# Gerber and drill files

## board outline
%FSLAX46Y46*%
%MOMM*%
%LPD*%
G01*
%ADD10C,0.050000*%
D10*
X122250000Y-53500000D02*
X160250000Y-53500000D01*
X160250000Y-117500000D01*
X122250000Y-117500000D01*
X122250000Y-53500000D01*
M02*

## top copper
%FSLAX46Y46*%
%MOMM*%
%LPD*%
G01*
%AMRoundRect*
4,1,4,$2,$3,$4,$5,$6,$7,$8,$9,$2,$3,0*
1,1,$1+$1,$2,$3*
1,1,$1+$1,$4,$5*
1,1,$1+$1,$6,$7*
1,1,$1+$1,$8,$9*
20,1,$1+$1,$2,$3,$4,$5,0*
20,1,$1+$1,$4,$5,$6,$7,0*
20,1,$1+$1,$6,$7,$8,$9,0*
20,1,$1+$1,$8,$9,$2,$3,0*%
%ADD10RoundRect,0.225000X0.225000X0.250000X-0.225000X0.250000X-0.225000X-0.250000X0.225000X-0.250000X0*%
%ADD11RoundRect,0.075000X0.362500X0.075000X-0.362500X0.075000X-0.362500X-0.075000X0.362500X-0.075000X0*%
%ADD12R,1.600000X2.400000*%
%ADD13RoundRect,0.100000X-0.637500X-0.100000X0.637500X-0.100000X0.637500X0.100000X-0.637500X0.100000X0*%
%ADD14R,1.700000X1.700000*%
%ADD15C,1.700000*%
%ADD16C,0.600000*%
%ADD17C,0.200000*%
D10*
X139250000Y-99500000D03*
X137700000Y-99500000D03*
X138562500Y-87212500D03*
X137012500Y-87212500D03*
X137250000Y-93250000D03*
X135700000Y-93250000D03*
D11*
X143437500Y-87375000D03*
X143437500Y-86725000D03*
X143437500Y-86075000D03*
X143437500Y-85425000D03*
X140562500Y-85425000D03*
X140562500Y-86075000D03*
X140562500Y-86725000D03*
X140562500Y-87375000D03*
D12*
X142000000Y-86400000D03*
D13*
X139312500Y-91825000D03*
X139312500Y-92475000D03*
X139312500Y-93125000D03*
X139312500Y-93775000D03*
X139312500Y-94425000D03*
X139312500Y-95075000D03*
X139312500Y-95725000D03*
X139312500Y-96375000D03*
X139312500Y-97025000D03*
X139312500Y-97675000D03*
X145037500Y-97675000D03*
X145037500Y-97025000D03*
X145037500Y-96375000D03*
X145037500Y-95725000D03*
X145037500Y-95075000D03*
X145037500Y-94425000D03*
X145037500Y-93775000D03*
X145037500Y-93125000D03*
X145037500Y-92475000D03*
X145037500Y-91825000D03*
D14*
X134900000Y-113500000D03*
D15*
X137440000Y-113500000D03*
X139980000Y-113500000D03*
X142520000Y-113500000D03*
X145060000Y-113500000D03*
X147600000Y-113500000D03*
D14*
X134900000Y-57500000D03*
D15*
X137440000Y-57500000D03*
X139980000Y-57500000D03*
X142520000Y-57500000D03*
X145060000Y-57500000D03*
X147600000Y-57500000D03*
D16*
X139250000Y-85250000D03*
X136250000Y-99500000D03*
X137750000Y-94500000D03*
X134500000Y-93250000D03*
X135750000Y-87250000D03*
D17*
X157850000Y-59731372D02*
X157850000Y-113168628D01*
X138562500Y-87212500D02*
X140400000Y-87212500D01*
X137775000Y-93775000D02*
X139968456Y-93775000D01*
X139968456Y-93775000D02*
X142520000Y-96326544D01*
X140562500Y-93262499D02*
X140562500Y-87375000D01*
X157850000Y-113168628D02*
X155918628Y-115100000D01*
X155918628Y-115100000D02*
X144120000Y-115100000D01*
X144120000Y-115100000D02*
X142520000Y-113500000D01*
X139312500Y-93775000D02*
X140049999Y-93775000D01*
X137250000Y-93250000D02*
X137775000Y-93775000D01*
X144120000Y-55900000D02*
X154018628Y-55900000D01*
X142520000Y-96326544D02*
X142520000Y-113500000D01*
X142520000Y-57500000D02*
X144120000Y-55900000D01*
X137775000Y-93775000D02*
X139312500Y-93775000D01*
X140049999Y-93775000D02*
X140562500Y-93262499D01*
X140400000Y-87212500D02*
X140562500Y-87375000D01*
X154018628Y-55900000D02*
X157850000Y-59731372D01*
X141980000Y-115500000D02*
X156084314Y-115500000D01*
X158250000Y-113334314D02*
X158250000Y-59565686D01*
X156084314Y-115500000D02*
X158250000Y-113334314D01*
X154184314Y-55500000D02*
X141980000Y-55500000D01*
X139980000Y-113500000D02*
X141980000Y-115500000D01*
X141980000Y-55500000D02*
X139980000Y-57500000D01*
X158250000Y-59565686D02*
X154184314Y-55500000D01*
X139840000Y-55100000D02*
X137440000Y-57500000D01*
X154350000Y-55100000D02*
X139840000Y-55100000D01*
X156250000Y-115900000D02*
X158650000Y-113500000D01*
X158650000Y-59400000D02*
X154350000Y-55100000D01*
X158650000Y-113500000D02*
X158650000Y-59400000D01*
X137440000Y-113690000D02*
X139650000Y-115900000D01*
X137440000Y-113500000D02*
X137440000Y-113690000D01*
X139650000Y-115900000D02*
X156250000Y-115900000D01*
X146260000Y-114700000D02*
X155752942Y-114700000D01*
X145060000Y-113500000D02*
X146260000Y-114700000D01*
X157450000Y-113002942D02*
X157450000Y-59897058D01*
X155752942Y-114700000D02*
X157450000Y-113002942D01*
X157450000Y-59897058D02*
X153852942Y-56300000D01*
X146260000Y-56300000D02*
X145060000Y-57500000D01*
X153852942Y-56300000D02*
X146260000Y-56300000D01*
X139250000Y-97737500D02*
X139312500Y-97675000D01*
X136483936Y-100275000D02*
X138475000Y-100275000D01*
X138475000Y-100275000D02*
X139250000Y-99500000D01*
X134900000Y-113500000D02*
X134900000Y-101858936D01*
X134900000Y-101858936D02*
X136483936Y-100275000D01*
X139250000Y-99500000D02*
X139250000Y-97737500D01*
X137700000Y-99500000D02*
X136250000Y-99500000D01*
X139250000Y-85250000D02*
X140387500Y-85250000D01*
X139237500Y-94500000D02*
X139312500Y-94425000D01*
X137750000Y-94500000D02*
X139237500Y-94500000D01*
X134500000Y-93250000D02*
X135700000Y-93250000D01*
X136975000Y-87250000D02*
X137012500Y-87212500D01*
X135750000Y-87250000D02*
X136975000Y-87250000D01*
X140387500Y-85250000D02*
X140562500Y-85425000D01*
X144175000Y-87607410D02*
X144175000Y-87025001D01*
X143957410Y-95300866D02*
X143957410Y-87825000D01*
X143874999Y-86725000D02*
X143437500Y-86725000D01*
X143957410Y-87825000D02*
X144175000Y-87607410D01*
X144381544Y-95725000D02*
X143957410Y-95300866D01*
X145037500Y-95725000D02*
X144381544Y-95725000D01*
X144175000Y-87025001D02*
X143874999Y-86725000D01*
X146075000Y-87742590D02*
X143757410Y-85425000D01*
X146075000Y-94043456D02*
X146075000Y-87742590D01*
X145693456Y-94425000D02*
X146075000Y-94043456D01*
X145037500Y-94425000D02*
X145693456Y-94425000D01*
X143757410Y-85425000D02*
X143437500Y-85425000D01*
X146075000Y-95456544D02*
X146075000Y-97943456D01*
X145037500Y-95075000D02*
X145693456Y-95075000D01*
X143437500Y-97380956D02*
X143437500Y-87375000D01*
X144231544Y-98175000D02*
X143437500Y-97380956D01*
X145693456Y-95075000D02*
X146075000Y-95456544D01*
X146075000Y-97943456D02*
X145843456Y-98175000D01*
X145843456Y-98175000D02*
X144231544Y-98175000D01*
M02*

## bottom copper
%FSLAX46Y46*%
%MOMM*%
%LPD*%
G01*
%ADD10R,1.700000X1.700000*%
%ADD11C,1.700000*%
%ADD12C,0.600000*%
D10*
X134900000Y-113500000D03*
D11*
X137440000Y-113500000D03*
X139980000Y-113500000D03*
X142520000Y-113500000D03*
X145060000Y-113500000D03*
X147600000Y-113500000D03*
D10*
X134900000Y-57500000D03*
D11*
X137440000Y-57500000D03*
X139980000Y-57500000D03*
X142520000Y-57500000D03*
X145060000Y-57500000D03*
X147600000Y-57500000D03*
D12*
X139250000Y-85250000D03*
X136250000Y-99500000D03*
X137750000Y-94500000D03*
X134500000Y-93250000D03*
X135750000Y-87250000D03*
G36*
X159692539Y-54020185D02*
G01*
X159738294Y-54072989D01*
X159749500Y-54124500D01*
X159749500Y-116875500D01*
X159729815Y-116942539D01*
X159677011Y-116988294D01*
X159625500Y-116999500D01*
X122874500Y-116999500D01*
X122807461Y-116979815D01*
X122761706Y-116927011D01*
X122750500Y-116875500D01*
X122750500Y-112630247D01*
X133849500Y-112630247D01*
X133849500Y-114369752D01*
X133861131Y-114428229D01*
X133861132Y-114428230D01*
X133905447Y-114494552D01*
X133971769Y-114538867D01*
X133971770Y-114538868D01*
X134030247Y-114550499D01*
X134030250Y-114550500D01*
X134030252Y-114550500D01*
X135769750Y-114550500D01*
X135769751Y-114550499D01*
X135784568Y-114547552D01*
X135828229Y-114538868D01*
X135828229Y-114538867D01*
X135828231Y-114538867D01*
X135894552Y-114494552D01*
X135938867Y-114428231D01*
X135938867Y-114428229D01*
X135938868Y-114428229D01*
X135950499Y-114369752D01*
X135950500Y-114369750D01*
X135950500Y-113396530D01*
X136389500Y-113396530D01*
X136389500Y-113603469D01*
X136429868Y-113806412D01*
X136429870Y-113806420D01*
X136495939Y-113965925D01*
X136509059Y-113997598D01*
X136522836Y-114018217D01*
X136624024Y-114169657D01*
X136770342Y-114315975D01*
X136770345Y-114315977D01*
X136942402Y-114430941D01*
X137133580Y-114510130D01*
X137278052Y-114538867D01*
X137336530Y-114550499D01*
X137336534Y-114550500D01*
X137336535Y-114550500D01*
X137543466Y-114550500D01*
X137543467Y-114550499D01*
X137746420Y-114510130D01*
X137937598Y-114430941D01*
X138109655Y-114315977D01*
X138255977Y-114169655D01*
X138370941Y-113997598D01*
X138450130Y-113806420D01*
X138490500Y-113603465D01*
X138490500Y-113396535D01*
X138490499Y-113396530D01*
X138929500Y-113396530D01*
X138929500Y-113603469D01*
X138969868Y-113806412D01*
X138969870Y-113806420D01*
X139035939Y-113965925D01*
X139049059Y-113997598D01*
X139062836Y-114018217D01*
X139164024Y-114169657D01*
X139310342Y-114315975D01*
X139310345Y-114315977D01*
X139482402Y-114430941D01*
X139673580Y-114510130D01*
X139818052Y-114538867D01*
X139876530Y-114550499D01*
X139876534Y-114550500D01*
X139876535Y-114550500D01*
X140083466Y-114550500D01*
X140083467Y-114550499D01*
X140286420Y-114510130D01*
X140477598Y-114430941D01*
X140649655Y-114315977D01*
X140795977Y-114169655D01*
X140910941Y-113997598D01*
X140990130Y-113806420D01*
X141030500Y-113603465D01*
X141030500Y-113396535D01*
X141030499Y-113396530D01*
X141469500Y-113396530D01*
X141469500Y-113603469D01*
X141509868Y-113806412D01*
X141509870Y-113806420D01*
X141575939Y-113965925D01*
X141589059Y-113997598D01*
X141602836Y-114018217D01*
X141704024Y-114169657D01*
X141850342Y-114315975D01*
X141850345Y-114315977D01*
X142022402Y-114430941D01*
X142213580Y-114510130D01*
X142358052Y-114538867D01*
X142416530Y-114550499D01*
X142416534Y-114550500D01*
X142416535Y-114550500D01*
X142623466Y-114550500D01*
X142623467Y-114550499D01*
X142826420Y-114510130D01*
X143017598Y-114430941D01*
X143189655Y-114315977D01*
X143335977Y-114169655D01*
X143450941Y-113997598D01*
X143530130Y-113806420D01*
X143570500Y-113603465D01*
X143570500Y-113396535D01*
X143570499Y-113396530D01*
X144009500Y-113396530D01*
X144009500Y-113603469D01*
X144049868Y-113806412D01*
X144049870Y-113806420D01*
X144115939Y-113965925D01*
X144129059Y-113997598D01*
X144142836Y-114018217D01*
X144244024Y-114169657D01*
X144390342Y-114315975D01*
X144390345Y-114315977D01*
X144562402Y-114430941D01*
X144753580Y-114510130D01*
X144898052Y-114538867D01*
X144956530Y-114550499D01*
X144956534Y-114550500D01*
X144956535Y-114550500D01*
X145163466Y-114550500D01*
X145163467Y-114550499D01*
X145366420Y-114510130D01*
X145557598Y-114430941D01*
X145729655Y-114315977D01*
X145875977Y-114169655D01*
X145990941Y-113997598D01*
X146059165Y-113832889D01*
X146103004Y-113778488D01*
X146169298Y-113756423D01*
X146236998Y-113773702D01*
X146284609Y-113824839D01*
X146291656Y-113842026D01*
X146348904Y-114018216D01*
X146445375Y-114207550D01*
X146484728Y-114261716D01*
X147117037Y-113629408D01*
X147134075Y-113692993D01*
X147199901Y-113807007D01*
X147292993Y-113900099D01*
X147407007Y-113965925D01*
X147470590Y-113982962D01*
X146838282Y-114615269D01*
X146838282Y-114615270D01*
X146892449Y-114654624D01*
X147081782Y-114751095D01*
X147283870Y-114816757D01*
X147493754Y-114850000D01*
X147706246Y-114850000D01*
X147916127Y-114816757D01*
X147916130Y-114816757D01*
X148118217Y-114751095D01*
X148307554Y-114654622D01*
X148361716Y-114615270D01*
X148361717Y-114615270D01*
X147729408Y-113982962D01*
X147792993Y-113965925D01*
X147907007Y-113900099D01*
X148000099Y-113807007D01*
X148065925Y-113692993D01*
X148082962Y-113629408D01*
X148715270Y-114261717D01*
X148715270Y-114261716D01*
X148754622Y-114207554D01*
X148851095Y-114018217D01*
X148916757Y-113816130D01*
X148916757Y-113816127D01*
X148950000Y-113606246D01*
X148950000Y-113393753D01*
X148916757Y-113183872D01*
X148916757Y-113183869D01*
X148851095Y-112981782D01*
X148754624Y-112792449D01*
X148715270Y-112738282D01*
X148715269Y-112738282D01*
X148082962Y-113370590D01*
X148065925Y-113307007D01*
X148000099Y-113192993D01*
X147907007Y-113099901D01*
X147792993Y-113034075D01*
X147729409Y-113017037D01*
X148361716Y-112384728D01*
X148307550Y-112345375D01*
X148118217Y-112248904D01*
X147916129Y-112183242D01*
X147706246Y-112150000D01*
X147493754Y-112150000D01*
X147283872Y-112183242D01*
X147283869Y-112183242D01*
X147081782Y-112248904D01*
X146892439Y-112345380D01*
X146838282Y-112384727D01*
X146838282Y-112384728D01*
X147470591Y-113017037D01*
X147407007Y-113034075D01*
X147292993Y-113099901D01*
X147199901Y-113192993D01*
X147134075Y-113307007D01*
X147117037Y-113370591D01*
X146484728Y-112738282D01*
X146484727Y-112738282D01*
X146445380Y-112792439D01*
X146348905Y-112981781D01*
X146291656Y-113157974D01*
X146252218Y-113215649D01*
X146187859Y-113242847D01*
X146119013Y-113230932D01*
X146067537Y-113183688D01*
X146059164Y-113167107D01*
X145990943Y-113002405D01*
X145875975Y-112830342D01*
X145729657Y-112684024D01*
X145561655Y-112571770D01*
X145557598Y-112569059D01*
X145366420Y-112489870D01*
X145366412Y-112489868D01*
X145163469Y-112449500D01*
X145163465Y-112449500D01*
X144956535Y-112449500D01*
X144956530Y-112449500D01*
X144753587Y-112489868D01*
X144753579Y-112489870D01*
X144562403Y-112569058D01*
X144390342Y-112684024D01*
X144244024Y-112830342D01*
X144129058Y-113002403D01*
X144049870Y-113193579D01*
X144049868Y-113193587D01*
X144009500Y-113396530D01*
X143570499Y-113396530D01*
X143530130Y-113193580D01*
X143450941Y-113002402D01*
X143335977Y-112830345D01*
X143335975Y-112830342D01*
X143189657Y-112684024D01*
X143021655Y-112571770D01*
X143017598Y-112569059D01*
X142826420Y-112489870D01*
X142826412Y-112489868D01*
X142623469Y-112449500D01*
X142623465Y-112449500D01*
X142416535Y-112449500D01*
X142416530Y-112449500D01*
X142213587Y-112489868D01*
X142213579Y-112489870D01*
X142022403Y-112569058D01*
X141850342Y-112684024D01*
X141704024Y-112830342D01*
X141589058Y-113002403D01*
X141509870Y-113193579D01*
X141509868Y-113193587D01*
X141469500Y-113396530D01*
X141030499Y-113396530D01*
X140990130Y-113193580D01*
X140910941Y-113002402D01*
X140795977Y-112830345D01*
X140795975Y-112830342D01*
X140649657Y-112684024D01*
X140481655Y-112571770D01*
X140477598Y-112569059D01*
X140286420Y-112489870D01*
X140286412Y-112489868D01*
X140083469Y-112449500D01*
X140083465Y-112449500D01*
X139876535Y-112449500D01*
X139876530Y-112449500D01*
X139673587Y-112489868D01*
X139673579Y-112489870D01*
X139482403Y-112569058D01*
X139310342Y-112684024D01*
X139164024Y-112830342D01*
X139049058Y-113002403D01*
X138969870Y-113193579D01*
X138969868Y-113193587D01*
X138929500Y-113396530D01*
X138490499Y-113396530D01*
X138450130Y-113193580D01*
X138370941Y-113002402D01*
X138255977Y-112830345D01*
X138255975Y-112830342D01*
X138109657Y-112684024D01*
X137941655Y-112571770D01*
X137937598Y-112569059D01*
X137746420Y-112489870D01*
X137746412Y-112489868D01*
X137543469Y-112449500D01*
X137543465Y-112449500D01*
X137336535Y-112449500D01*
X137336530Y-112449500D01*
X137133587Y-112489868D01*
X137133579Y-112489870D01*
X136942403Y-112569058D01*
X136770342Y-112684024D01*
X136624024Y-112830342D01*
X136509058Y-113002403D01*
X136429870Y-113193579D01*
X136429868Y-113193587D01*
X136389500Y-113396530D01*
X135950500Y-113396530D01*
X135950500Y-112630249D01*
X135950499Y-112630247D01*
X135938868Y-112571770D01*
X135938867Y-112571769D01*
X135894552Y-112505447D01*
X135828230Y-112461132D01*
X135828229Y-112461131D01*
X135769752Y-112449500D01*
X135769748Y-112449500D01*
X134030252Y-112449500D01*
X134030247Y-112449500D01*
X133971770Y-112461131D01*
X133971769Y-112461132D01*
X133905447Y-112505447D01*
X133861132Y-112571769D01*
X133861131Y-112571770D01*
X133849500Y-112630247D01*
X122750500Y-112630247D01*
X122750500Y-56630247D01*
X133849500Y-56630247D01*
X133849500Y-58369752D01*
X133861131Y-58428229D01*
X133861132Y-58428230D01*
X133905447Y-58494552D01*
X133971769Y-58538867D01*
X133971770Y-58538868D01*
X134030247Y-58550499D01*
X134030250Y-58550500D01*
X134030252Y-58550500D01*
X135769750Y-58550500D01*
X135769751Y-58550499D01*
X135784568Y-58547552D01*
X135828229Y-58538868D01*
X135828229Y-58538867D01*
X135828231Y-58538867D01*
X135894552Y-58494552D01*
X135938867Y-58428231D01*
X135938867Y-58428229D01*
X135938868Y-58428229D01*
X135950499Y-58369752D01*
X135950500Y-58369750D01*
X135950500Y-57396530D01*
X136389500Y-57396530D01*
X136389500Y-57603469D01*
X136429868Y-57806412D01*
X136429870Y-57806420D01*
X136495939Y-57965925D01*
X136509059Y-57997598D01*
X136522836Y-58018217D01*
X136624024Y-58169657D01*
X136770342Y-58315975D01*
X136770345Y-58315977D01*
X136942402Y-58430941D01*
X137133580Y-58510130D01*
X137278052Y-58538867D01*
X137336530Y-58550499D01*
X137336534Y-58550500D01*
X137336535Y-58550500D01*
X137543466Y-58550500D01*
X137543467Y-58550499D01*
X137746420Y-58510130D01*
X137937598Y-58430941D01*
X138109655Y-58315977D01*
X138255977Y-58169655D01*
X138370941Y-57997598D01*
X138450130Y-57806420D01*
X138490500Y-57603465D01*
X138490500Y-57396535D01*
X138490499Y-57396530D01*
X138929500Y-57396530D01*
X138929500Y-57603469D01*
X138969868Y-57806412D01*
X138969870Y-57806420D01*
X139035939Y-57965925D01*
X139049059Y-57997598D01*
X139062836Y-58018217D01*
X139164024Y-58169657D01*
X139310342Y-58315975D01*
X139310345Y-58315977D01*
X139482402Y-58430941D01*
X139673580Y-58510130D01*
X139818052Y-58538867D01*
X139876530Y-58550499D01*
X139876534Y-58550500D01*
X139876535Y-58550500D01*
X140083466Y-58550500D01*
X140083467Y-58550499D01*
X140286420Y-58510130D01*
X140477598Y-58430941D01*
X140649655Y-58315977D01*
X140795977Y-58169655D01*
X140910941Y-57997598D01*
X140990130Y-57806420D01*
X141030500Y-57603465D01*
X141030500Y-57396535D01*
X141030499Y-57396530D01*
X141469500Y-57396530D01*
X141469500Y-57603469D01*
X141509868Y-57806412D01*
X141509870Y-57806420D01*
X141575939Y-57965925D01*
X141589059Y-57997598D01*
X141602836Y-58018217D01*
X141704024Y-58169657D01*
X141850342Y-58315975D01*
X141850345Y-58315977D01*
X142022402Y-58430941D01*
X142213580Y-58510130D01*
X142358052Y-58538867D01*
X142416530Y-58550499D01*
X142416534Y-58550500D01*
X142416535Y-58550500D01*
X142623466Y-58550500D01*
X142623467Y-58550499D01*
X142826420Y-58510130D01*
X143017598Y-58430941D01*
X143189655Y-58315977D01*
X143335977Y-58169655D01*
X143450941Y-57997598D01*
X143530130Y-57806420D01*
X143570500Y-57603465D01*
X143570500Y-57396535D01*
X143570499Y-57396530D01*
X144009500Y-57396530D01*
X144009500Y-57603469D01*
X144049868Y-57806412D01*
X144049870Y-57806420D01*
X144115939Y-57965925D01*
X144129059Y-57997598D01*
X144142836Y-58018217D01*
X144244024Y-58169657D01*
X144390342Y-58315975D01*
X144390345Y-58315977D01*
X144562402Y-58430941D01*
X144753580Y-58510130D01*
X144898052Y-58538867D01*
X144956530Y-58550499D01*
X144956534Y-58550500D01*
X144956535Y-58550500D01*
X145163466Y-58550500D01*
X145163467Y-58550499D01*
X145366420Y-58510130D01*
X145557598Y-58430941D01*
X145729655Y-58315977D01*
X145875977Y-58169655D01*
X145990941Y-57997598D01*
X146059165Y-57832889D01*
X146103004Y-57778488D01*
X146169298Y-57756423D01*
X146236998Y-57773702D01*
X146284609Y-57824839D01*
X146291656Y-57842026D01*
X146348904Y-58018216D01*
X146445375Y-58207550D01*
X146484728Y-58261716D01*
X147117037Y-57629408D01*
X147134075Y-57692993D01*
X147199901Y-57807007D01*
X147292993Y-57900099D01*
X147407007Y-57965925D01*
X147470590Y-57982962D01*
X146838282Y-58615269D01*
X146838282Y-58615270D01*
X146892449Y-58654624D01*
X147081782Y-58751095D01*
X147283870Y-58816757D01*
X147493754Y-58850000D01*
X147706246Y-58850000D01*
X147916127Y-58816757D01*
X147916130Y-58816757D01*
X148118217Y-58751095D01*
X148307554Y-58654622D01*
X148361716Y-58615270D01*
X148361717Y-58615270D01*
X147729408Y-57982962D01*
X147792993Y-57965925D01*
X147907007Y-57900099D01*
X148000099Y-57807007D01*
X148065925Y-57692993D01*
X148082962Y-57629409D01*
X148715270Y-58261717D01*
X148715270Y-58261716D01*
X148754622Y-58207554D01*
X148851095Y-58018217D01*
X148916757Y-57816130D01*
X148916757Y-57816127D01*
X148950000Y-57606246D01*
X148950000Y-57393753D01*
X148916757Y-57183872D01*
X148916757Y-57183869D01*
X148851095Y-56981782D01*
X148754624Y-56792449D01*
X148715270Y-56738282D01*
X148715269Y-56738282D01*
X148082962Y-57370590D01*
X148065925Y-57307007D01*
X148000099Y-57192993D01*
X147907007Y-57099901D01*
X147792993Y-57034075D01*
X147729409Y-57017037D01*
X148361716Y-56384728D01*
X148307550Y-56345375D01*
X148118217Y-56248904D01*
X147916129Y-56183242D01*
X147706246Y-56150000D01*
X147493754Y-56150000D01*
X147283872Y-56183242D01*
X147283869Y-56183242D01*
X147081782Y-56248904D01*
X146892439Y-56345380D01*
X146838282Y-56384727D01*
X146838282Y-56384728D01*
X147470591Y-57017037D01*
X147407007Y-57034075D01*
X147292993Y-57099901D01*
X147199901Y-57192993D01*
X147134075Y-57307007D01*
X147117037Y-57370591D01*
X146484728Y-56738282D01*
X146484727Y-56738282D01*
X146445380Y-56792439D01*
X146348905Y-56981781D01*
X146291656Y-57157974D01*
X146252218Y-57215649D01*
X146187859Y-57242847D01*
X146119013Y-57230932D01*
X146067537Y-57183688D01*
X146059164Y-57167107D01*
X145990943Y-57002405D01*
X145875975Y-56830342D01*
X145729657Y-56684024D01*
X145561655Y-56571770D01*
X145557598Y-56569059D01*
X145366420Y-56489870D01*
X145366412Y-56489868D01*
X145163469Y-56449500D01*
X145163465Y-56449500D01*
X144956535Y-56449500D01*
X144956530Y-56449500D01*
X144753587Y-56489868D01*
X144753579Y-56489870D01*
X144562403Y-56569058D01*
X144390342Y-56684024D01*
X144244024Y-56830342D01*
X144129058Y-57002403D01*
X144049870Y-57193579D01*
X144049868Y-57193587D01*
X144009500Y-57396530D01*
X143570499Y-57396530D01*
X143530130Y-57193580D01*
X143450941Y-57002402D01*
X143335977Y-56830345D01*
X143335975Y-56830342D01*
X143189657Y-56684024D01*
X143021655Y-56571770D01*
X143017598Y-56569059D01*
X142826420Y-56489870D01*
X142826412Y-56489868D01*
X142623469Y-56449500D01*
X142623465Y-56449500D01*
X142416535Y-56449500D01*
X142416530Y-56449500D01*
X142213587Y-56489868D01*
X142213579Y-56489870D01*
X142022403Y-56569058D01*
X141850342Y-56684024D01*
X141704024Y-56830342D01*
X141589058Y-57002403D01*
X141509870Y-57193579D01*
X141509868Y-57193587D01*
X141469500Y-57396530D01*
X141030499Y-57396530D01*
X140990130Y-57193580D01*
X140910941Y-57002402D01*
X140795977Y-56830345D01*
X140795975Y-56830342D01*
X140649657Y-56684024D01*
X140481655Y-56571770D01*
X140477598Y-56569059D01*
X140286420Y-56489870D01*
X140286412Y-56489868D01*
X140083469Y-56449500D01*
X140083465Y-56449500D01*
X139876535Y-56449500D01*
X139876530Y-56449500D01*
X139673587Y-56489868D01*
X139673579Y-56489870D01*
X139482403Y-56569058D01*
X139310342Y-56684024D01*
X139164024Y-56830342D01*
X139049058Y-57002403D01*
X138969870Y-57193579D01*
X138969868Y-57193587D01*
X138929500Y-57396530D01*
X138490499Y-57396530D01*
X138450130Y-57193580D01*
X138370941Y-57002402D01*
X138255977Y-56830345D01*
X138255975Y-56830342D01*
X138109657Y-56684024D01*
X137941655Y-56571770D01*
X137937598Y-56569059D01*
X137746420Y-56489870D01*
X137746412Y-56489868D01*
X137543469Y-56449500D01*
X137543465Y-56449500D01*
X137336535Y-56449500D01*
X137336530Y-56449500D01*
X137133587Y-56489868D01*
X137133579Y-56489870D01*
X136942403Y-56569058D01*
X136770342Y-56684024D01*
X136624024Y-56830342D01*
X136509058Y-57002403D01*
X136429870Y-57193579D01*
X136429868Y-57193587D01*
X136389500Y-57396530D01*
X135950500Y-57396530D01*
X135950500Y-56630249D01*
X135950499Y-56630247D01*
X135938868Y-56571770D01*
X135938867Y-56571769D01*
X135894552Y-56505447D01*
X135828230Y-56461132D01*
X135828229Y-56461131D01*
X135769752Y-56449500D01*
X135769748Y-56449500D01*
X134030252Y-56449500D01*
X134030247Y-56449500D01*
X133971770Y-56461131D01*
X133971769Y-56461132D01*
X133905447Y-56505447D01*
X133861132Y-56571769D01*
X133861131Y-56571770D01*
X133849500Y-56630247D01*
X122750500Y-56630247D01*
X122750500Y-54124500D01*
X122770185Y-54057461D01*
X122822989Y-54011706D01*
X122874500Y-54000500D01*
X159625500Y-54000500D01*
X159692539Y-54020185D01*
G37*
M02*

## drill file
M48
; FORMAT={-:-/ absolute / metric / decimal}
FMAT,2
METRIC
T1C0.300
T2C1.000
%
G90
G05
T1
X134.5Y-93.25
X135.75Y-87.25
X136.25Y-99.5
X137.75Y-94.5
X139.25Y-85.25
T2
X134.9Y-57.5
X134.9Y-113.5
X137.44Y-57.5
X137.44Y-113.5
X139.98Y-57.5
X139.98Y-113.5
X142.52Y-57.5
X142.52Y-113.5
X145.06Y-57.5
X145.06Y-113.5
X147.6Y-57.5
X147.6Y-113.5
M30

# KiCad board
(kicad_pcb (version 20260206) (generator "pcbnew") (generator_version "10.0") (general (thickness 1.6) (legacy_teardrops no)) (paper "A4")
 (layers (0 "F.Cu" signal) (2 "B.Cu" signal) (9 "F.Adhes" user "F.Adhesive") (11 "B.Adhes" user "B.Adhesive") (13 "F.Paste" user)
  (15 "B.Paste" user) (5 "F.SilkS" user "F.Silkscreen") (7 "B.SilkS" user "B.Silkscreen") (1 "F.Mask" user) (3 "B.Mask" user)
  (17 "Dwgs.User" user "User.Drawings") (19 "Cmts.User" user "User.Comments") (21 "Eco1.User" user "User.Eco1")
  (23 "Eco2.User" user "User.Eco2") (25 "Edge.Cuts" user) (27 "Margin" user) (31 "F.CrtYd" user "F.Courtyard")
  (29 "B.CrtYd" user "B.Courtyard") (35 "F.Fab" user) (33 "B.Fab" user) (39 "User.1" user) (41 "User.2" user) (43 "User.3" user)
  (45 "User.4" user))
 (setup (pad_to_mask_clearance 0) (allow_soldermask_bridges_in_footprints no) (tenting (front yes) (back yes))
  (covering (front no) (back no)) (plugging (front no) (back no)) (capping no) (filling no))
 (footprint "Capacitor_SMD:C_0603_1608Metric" (layer "F.Cu") (at 138.475 99.5 180)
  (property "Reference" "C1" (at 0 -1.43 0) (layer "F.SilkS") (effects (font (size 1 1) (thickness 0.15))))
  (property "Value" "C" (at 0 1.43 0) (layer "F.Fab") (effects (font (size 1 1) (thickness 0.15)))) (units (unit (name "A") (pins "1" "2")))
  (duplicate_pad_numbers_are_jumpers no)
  (pad "1" smd roundrect (at -0.775 0 180) (size 0.9 0.95) (layers "F.Cu" "F.Mask" "F.Paste") (roundrect_rratio 0.25) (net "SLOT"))
  (pad "2" smd roundrect (at 0.775 0 180) (size 0.9 0.95) (layers "F.Cu" "F.Mask" "F.Paste") (roundrect_rratio 0.25) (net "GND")))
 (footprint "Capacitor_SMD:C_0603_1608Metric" (layer "F.Cu") (at 137.7875 87.2125 180)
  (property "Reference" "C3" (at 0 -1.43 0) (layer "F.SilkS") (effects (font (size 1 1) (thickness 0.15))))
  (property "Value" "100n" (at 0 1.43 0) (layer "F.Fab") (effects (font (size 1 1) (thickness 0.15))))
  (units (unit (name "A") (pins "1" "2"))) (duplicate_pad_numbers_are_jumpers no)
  (pad "1" smd roundrect (at -0.775 0 180) (size 0.9 0.95) (layers "F.Cu" "F.Mask" "F.Paste") (roundrect_rratio 0.25) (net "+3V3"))
  (pad "2" smd roundrect (at 0.775 0 180) (size 0.9 0.95) (layers "F.Cu" "F.Mask" "F.Paste") (roundrect_rratio 0.25) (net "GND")))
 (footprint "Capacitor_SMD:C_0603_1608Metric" (layer "F.Cu") (at 136.475 93.25 180)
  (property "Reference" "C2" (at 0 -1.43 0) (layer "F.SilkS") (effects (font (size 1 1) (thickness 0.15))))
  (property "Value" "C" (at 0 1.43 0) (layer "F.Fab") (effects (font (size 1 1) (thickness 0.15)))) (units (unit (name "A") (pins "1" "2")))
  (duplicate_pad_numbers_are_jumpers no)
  (pad "1" smd roundrect (at -0.775 0 180) (size 0.9 0.95) (layers "F.Cu" "F.Mask" "F.Paste") (roundrect_rratio 0.25) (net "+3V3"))
  (pad "2" smd roundrect (at 0.775 0 180) (size 0.9 0.95) (layers "F.Cu" "F.Mask" "F.Paste") (roundrect_rratio 0.25) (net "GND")))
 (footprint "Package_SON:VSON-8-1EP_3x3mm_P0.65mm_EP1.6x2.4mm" (layer "F.Cu") (at 142 86.4 180)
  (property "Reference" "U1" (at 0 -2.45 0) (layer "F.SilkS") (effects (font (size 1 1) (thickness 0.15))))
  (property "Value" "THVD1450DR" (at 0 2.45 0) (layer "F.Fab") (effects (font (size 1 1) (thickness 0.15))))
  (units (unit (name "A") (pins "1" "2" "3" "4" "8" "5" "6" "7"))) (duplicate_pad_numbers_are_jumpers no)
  (pad "" smd roundrect (at 0 -0.6 180) (size 1.29 0.97) (layers "F.Paste") (roundrect_rratio 0.25))
  (pad "" smd roundrect (at 0 0.6 180) (size 1.29 0.97) (layers "F.Paste") (roundrect_rratio 0.25))
  (pad "1" smd roundrect (at -1.4375 -0.975 180) (size 0.875 0.3) (layers "F.Cu" "F.Mask" "F.Paste") (roundrect_rratio 0.25) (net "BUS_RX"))
  (pad "2" smd roundrect (at -1.4375 -0.325 180) (size 0.875 0.3) (layers "F.Cu" "F.Mask" "F.Paste") (roundrect_rratio 0.25) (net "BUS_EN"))
  (pad "3" smd roundrect (at -1.4375 0.325 180) (size 0.875 0.3) (layers "F.Cu" "F.Mask" "F.Paste") (roundrect_rratio 0.25) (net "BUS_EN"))
  (pad "4" smd roundrect (at -1.4375 0.975 180) (size 0.875 0.3) (layers "F.Cu" "F.Mask" "F.Paste") (roundrect_rratio 0.25) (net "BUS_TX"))
  (pad "5" smd roundrect (at 1.4375 0.975 180) (size 0.875 0.3) (layers "F.Cu" "F.Mask" "F.Paste") (roundrect_rratio 0.25) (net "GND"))
  (pad "6" smd roundrect (at 1.4375 0.325 180) (size 0.875 0.3) (layers "F.Cu" "F.Mask" "F.Paste") (roundrect_rratio 0.25) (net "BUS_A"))
  (pad "7" smd roundrect (at 1.4375 -0.325 180) (size 0.875 0.3) (layers "F.Cu" "F.Mask" "F.Paste") (roundrect_rratio 0.25) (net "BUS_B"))
  (pad "8" smd roundrect (at 1.4375 -0.975 180) (size 0.875 0.3) (layers "F.Cu" "F.Mask" "F.Paste") (roundrect_rratio 0.25) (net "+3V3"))
  (pad "9" smd rect (at 0 0 180) (size 1.6 2.4) (layers "F.Cu" "F.Mask") (zone_connect 2)))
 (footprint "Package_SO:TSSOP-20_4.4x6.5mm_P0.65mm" (layer "F.Cu") (at 142.175 94.75)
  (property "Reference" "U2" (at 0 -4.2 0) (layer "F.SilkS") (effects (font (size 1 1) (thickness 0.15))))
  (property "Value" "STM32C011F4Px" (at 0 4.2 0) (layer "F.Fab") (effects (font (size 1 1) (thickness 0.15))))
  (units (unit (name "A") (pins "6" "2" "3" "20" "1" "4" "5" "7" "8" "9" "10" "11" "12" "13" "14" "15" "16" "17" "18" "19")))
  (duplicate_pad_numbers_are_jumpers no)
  (pad "1" smd roundrect (at -2.8625 -2.925) (size 1.475 0.4) (layers "F.Cu" "F.Mask" "F.Paste") (roundrect_rratio 0.25)
   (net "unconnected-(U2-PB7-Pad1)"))
  (pad "2" smd roundrect (at -2.8625 -2.275) (size 1.475 0.4) (layers "F.Cu" "F.Mask" "F.Paste") (roundrect_rratio 0.25)
   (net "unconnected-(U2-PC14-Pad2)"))
  (pad "3" smd roundrect (at -2.8625 -1.625) (size 1.475 0.4) (layers "F.Cu" "F.Mask" "F.Paste") (roundrect_rratio 0.25)
   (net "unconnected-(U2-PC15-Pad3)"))
  (pad "4" smd roundrect (at -2.8625 -0.975) (size 1.475 0.4) (layers "F.Cu" "F.Mask" "F.Paste") (roundrect_rratio 0.25) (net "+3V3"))
  (pad "5" smd roundrect (at -2.8625 -0.325) (size 1.475 0.4) (layers "F.Cu" "F.Mask" "F.Paste") (roundrect_rratio 0.25) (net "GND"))
  (pad "6" smd roundrect (at -2.8625 0.325) (size 1.475 0.4) (layers "F.Cu" "F.Mask" "F.Paste") (roundrect_rratio 0.25)
   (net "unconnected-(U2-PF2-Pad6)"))
  (pad "7" smd roundrect (at -2.8625 0.975) (size 1.475 0.4) (layers "F.Cu" "F.Mask" "F.Paste") (roundrect_rratio 0.25)
   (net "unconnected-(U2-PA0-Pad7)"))
  (pad "8" smd roundrect (at -2.8625 1.625) (size 1.475 0.4) (layers "F.Cu" "F.Mask" "F.Paste") (roundrect_rratio 0.25)
   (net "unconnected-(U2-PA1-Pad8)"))
  (pad "9" smd roundrect (at -2.8625 2.275) (size 1.475 0.4) (layers "F.Cu" "F.Mask" "F.Paste") (roundrect_rratio 0.25)
   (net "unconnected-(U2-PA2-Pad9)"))
  (pad "10" smd roundrect (at -2.8625 2.925) (size 1.475 0.4) (layers "F.Cu" "F.Mask" "F.Paste") (roundrect_rratio 0.25) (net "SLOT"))
  (pad "11" smd roundrect (at 2.8625 2.925) (size 1.475 0.4) (layers "F.Cu" "F.Mask" "F.Paste") (roundrect_rratio 0.25)
   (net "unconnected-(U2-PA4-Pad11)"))
  (pad "12" smd roundrect (at 2.8625 2.275) (size 1.475 0.4) (layers "F.Cu" "F.Mask" "F.Paste") (roundrect_rratio 0.25)
   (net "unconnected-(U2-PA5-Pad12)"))
  (pad "13" smd roundrect (at 2.8625 1.625) (size 1.475 0.4) (layers "F.Cu" "F.Mask" "F.Paste") (roundrect_rratio 0.25)
   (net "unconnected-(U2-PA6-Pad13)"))
  (pad "14" smd roundrect (at 2.8625 0.975) (size 1.475 0.4) (layers "F.Cu" "F.Mask" "F.Paste") (roundrect_rratio 0.25) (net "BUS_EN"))
  (pad "15" smd roundrect (at 2.8625 0.325) (size 1.475 0.4) (layers "F.Cu" "F.Mask" "F.Paste") (roundrect_rratio 0.25) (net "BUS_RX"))
  (pad "16" smd roundrect (at 2.8625 -0.325) (size 1.475 0.4) (layers "F.Cu" "F.Mask" "F.Paste") (roundrect_rratio 0.25) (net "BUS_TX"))
  (pad "17" smd roundrect (at 2.8625 -0.975) (size 1.475 0.4) (layers "F.Cu" "F.Mask" "F.Paste") (roundrect_rratio 0.25)
   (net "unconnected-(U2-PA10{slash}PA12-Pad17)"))
  (pad "18" smd roundrect (at 2.8625 -1.625) (size 1.475 0.4) (layers "F.Cu" "F.Mask" "F.Paste") (roundrect_rratio 0.25)
   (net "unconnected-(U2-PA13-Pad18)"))
  (pad "19" smd roundrect (at 2.8625 -2.275) (size 1.475 0.4) (layers "F.Cu" "F.Mask" "F.Paste") (roundrect_rratio 0.25)
   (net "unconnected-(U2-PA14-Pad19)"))
  (pad "20" smd roundrect (at 2.8625 -2.925) (size 1.475 0.4) (layers "F.Cu" "F.Mask" "F.Paste") (roundrect_rratio 0.25)
   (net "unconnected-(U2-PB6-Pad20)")))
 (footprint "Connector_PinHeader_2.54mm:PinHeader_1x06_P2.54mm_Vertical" (layer "B.Cu") (at 134.9 113.5 -90)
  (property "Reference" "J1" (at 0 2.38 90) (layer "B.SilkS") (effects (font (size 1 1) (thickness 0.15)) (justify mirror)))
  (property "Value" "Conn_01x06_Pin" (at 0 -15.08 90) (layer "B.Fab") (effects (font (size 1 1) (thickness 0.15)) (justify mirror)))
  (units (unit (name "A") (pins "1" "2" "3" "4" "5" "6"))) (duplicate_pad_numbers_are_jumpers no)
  (pad "1" thru_hole rect (at 0 0 270) (size 1.7 1.7) (drill 1) (layers "*.Cu" "*.Mask") (remove_unused_layers no) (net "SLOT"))
  (pad "2" thru_hole circle (at 0 -2.54 270) (size 1.7 1.7) (drill 1) (layers "*.Cu" "*.Mask") (remove_unused_layers no) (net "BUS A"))
  (pad "3" thru_hole circle (at 0 -5.08 270) (size 1.7 1.7) (drill 1) (layers "*.Cu" "*.Mask") (remove_unused_layers no) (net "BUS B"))
  (pad "4" thru_hole circle (at 0 -7.62 270) (size 1.7 1.7) (drill 1) (layers "*.Cu" "*.Mask") (remove_unused_layers no) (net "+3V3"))
  (pad "5" thru_hole circle (at 0 -10.16 270) (size 1.7 1.7) (drill 1) (layers "*.Cu" "*.Mask") (remove_unused_layers no) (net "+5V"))
  (pad "6" thru_hole circle (at 0 -12.7 270) (size 1.7 1.7) (drill 1) (layers "*.Cu" "*.Mask") (remove_unused_layers no) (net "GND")))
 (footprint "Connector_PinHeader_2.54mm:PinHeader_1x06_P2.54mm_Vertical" (layer "B.Cu") (at 134.9 57.5 -90)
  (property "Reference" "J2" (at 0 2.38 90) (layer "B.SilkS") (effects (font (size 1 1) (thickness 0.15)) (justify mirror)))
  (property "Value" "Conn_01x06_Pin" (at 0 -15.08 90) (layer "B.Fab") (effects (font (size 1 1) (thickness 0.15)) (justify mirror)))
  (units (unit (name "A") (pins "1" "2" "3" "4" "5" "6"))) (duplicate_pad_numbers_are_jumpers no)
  (pad "1" thru_hole rect (at 0 0 270) (size 1.7 1.7) (drill 1) (layers "*.Cu" "*.Mask") (remove_unused_layers no) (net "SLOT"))
  (pad "2" thru_hole circle (at 0 -2.54 270) (size 1.7 1.7) (drill 1) (layers "*.Cu" "*.Mask") (remove_unused_layers no) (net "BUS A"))
  (pad "3" thru_hole circle (at 0 -5.08 270) (size 1.7 1.7) (drill 1) (layers "*.Cu" "*.Mask") (remove_unused_layers no) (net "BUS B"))
  (pad "4" thru_hole circle (at 0 -7.62 270) (size 1.7 1.7) (drill 1) (layers "*.Cu" "*.Mask") (remove_unused_layers no) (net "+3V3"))
  (pad "5" thru_hole circle (at 0 -10.16 270) (size 1.7 1.7) (drill 1) (layers "*.Cu" "*.Mask") (remove_unused_layers no) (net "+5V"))
  (pad "6" thru_hole circle (at 0 -12.7 270) (size 1.7 1.7) (drill 1) (layers "*.Cu" "*.Mask") (remove_unused_layers no) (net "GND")))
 (gr_rect (start 122.25 53.5) (end 160.25 117.5) (stroke (width 0.05) (type solid)) (fill no) (layer "Edge.Cuts"))
 (segment (start 157.85 59.731372) (end 157.85 113.168628) (width 0.2) (layer "F.Cu") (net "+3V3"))
 (segment (start 138.5625 87.2125) (end 140.4 87.2125) (width 0.2) (layer "F.Cu") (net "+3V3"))
 (segment (start 137.775 93.775) (end 139.968456 93.775) (width 0.2) (layer "F.Cu") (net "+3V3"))
 (segment (start 139.968456 93.775) (end 142.52 96.326544) (width 0.2) (layer "F.Cu") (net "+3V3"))
 (segment (start 140.5625 93.262499) (end 140.5625 87.375) (width 0.2) (layer "F.Cu") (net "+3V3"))
 (segment (start 157.85 113.168628) (end 155.918628 115.1) (width 0.2) (layer "F.Cu") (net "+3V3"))
 (segment (start 155.918628 115.1) (end 144.12 115.1) (width 0.2) (layer "F.Cu") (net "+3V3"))
 (segment (start 144.12 115.1) (end 142.52 113.5) (width 0.2) (layer "F.Cu") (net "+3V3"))
 (segment (start 139.3125 93.775) (end 140.049999 93.775) (width 0.2) (layer "F.Cu") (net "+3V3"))
 (segment (start 137.25 93.25) (end 137.775 93.775) (width 0.2) (layer "F.Cu") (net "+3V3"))
 (segment (start 144.12 55.9) (end 154.018628 55.9) (width 0.2) (layer "F.Cu") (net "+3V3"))
 (segment (start 142.52 96.326544) (end 142.52 113.5) (width 0.2) (layer "F.Cu") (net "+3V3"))
 (segment (start 142.52 57.5) (end 144.12 55.9) (width 0.2) (layer "F.Cu") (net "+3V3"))
 (segment (start 137.775 93.775) (end 139.3125 93.775) (width 0.2) (layer "F.Cu") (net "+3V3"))
 (segment (start 140.049999 93.775) (end 140.5625 93.262499) (width 0.2) (layer "F.Cu") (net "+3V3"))
 (segment (start 140.4 87.2125) (end 140.5625 87.375) (width 0.2) (layer "F.Cu") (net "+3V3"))
 (segment (start 154.018628 55.9) (end 157.85 59.731372) (width 0.2) (layer "F.Cu") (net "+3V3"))
 (segment (start 141.98 115.5) (end 156.084314 115.5) (width 0.2) (layer "F.Cu") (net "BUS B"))
 (segment (start 158.25 113.334314) (end 158.25 59.565686) (width 0.2) (layer "F.Cu") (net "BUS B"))
 (segment (start 156.084314 115.5) (end 158.25 113.334314) (width 0.2) (layer "F.Cu") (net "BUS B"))
 (segment (start 154.184314 55.5) (end 141.98 55.5) (width 0.2) (layer "F.Cu") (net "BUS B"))
 (segment (start 139.98 113.5) (end 141.98 115.5) (width 0.2) (layer "F.Cu") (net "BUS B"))
 (segment (start 141.98 55.5) (end 139.98 57.5) (width 0.2) (layer "F.Cu") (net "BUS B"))
 (segment (start 158.25 59.565686) (end 154.184314 55.5) (width 0.2) (layer "F.Cu") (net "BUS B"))
 (segment (start 139.84 55.1) (end 137.44 57.5) (width 0.2) (layer "F.Cu") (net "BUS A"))
 (segment (start 154.35 55.1) (end 139.84 55.1) (width 0.2) (layer "F.Cu") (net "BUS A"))
 (segment (start 156.25 115.9) (end 158.65 113.5) (width 0.2) (layer "F.Cu") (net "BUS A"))
 (segment (start 158.65 59.4) (end 154.35 55.1) (width 0.2) (layer "F.Cu") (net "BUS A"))
 (segment (start 158.65 113.5) (end 158.65 59.4) (width 0.2) (layer "F.Cu") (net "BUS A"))
 (segment (start 137.44 113.69) (end 139.65 115.9) (width 0.2) (layer "F.Cu") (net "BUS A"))
 (segment (start 137.44 113.5) (end 137.44 113.69) (width 0.2) (layer "F.Cu") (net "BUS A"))
 (segment (start 139.65 115.9) (end 156.25 115.9) (width 0.2) (layer "F.Cu") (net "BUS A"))
 (segment (start 146.26 114.7) (end 155.752942 114.7) (width 0.2) (layer "F.Cu") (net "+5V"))
 (segment (start 145.06 113.5) (end 146.26 114.7) (width 0.2) (layer "F.Cu") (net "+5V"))
 (segment (start 157.45 113.002942) (end 157.45 59.897058) (width 0.2) (layer "F.Cu") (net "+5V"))
 (segment (start 155.752942 114.7) (end 157.45 113.002942) (width 0.2) (layer "F.Cu") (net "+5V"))
 (segment (start 157.45 59.897058) (end 153.852942 56.3) (width 0.2) (layer "F.Cu") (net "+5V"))
 (segment (start 146.26 56.3) (end 145.06 57.5) (width 0.2) (layer "F.Cu") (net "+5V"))
 (segment (start 153.852942 56.3) (end 146.26 56.3) (width 0.2) (layer "F.Cu") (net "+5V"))
 (segment (start 139.25 97.7375) (end 139.3125 97.675) (width 0.2) (layer "F.Cu") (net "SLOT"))
 (segment (start 136.483936 100.275) (end 138.475 100.275) (width 0.2) (layer "F.Cu") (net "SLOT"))
 (segment (start 138.475 100.275) (end 139.25 99.5) (width 0.2) (layer "F.Cu") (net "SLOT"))
 (segment (start 134.9 113.5) (end 134.9 101.858936) (width 0.2) (layer "F.Cu") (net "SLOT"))
 (segment (start 134.9 101.858936) (end 136.483936 100.275) (width 0.2) (layer "F.Cu") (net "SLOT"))
 (segment (start 139.25 99.5) (end 139.25 97.7375) (width 0.2) (layer "F.Cu") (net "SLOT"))
 (segment (start 137.7 99.5) (end 136.25 99.5) (width 0.2) (layer "F.Cu") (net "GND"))
 (segment (start 139.25 85.25) (end 140.3875 85.25) (width 0.2) (layer "F.Cu") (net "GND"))
 (segment (start 139.2375 94.5) (end 139.3125 94.425) (width 0.2) (layer "F.Cu") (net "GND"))
 (segment (start 137.75 94.5) (end 139.2375 94.5) (width 0.2) (layer "F.Cu") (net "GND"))
 (segment (start 134.5 93.25) (end 135.7 93.25) (width 0.2) (layer "F.Cu") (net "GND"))
 (segment (start 136.975 87.25) (end 137.0125 87.2125) (width 0.2) (layer "F.Cu") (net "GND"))
 (segment (start 135.75 87.25) (end 136.975 87.25) (width 0.2) (layer "F.Cu") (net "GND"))
 (segment (start 140.3875 85.25) (end 140.5625 85.425) (width 0.2) (layer "F.Cu") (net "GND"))
 (via (at 139.25 85.25) (size 0.6) (drill 0.3) (layers "F.Cu" "B.Cu") (free yes) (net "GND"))
 (via (at 136.25 99.5) (size 0.6) (drill 0.3) (layers "F.Cu" "B.Cu") (free yes) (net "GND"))
 (via (at 137.75 94.5) (size 0.6) (drill 0.3) (layers "F.Cu" "B.Cu") (free yes) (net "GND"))
 (via (at 134.5 93.25) (size 0.6) (drill 0.3) (layers "F.Cu" "B.Cu") (free yes) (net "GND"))
 (via (at 135.75 87.25) (size 0.6) (drill 0.3) (layers "F.Cu" "B.Cu") (free yes) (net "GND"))
 (segment (start 144.175 87.60741) (end 144.175 87.025001) (width 0.2) (layer "F.Cu") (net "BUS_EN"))
 (segment (start 143.95741 95.300866) (end 143.95741 87.825) (width 0.2) (layer "F.Cu") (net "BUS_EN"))
 (segment (start 143.874999 86.725) (end 143.4375 86.725) (width 0.2) (layer "F.Cu") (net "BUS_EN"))
 (segment (start 143.95741 87.825) (end 144.175 87.60741) (width 0.2) (layer "F.Cu") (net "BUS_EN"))
 (segment (start 144.381544 95.725) (end 143.95741 95.300866) (width 0.2) (layer "F.Cu") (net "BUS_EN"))
 (segment (start 145.0375 95.725) (end 144.381544 95.725) (width 0.2) (layer "F.Cu") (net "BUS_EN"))
 (segment (start 144.175 87.025001) (end 143.874999 86.725) (width 0.2) (layer "F.Cu") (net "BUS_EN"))
 (segment (start 146.075 87.74259) (end 143.75741 85.425) (width 0.2) (layer "F.Cu") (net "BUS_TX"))
 (segment (start 146.075 94.043456) (end 146.075 87.74259) (width 0.2) (layer "F.Cu") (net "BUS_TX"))
 (segment (start 145.693456 94.425) (end 146.075 94.043456) (width 0.2) (layer "F.Cu") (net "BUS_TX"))
 (segment (start 145.0375 94.425) (end 145.693456 94.425) (width 0.2) (layer "F.Cu") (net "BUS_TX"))
 (segment (start 143.75741 85.425) (end 143.4375 85.425) (width 0.2) (layer "F.Cu") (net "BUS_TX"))
 (segment (start 146.075 95.456544) (end 146.075 97.943456) (width 0.2) (layer "F.Cu") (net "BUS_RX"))
 (segment (start 145.0375 95.075) (end 145.693456 95.075) (width 0.2) (layer "F.Cu") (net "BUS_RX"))
 (segment (start 143.4375 97.380956) (end 143.4375 87.375) (width 0.2) (layer "F.Cu") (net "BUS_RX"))
 (segment (start 144.231544 98.175) (end 143.4375 97.380956) (width 0.2) (layer "F.Cu") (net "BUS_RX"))
 (segment (start 145.693456 95.075) (end 146.075 95.456544) (width 0.2) (layer "F.Cu") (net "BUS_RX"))
 (segment (start 146.075 97.943456) (end 145.843456 98.175) (width 0.2) (layer "F.Cu") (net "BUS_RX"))
 (segment (start 145.843456 98.175) (end 144.231544 98.175) (width 0.2) (layer "F.Cu") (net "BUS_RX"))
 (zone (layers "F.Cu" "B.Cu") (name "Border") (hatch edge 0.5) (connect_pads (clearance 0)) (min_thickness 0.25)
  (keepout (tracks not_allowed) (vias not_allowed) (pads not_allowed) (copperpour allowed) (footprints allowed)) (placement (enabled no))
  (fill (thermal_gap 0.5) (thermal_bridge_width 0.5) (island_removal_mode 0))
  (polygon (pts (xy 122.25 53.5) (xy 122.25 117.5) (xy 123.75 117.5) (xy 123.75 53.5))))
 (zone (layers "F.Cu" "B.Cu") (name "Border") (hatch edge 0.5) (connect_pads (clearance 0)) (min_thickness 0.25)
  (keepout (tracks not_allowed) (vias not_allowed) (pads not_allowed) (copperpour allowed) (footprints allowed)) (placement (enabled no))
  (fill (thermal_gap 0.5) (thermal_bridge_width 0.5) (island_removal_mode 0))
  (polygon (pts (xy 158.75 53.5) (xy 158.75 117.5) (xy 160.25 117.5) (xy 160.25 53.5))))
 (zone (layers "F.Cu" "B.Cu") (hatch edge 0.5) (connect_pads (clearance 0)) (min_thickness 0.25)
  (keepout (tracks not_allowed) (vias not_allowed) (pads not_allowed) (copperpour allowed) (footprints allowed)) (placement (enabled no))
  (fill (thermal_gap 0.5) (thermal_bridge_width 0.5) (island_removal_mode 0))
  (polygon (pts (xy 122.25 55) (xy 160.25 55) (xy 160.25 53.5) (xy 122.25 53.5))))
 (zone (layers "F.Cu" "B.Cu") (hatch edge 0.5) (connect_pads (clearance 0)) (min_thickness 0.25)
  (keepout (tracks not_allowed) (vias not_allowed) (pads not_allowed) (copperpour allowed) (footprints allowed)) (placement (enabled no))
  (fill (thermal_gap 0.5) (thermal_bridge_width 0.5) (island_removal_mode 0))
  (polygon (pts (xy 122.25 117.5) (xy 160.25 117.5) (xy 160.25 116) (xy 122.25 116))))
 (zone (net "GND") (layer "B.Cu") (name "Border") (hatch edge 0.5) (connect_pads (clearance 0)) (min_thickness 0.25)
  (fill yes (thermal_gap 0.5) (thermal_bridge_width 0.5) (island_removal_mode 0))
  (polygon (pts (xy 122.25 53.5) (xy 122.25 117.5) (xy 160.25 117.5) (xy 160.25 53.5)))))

